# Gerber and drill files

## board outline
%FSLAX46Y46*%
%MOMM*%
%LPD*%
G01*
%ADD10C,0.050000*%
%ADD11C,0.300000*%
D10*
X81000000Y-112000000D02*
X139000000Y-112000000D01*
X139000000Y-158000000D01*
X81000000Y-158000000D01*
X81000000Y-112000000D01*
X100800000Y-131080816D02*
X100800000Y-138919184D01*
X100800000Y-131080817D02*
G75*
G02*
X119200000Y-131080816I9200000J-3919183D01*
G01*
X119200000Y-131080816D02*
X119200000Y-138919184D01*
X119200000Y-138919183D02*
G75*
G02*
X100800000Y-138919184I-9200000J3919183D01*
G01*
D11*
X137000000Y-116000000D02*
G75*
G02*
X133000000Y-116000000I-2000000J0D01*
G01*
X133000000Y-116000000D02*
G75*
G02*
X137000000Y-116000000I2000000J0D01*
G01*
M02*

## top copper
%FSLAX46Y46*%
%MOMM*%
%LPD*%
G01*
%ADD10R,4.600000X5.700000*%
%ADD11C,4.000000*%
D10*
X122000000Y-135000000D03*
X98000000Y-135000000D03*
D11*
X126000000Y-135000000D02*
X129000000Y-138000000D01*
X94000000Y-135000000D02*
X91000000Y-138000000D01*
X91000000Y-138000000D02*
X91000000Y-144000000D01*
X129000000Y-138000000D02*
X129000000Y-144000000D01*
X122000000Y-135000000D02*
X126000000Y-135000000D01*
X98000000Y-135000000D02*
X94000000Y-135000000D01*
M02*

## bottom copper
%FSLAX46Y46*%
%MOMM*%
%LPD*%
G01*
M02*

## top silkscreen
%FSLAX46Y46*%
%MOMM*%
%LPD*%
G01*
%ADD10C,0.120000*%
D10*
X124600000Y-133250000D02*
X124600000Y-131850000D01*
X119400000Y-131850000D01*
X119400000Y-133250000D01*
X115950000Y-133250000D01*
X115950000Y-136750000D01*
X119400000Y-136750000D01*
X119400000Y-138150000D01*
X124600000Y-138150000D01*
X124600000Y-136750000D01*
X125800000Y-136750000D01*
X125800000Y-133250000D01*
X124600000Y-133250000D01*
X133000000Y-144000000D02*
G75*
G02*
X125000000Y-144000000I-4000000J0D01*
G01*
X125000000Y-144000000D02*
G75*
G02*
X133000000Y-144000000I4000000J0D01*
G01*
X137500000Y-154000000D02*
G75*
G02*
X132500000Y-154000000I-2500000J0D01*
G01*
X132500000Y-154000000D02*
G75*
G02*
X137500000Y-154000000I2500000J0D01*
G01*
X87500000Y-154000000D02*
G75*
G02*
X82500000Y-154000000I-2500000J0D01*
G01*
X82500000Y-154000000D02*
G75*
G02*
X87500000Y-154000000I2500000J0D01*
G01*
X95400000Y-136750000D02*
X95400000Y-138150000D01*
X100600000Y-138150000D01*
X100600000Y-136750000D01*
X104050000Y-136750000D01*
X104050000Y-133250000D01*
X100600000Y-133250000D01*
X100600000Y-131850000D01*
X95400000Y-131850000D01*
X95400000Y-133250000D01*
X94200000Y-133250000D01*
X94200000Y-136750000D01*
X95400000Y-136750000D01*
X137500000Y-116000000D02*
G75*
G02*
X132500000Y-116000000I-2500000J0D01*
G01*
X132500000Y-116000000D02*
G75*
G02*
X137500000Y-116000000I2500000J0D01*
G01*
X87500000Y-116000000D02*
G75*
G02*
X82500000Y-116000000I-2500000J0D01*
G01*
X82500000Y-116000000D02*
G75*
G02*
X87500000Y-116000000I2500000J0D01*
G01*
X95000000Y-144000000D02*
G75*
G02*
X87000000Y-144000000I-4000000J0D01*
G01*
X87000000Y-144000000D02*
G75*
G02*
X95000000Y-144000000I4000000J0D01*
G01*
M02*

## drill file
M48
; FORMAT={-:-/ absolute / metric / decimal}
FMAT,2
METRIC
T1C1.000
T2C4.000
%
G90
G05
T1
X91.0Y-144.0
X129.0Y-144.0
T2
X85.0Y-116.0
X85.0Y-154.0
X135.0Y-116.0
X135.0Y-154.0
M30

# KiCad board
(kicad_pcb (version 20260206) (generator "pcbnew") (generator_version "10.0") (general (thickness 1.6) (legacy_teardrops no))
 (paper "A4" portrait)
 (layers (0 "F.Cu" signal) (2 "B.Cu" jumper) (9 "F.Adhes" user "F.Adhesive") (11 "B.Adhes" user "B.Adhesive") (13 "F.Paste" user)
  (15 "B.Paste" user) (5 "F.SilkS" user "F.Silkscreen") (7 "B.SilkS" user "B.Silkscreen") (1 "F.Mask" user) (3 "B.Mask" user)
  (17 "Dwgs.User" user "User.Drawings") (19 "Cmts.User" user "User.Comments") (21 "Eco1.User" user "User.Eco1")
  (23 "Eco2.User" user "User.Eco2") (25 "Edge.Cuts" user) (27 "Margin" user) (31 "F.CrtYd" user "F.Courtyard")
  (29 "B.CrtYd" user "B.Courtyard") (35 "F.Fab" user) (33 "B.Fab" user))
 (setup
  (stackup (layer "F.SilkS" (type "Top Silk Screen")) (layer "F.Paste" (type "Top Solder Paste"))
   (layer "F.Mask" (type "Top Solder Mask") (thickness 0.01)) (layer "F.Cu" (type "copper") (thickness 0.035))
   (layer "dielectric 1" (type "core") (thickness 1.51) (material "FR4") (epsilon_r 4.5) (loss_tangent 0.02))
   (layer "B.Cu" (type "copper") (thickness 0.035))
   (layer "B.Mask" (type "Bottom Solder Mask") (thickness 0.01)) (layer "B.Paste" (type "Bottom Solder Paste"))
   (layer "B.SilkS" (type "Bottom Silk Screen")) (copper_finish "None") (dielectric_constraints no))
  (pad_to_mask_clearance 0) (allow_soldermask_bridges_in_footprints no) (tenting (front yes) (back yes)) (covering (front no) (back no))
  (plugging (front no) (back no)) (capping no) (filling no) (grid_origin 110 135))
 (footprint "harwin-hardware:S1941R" (layer "F.Cu") (at 122 135)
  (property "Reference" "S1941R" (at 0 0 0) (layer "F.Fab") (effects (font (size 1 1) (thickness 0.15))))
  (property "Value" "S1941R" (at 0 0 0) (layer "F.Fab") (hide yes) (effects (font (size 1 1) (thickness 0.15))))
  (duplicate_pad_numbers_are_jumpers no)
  (fp_poly
   (pts (xy 2.6 -1.75) (xy 2.6 -3.15) (xy -2.6 -3.15) (xy -2.6 -1.75) (xy -6.05 -1.75) (xy -6.05 1.75) (xy -2.6 1.75) (xy -2.6 3.15)
    (xy 2.6 3.15) (xy 2.6 1.75) (xy 3.8 1.75) (xy 3.8 -1.75))
   (stroke (width 0.12) (type solid)) (fill no) (layer "F.SilkS"))
  (pad "1" smd rect (at 0 0) (size 4.6 5.7) (layers "F.Cu" "F.Mask" "F.Paste")))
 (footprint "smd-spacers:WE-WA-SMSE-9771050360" (layer "F.Cu") (at 129 144)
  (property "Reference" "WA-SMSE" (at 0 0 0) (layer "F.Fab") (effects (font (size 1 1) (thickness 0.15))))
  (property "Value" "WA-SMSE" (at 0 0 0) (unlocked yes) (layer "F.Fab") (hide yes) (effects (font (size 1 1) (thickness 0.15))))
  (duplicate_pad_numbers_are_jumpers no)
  (fp_circle (center 0 0) (end 4 0) (stroke (width 0.12) (type default)) (fill no) (layer "F.SilkS"))
  (pad "" np_thru_hole circle (at 0 0) (size 1 1) (drill 1) (layers "*.Cu" "*.Mask")))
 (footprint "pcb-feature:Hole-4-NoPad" (layer "F.Cu") (at 135 154)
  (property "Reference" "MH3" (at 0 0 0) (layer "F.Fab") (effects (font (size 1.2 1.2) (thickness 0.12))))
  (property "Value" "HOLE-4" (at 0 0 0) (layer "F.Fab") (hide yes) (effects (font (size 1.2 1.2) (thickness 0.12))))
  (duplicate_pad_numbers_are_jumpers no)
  (fp_circle (center 0 0) (end 2.5 0) (stroke (width 0.12) (type solid)) (fill no) (layer "F.SilkS"))
  (pad "" np_thru_hole circle (at 0 0) (size 4 4) (drill 4) (layers "*.Cu" "*.Mask")))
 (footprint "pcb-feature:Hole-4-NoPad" (layer "F.Cu") (at 85 154)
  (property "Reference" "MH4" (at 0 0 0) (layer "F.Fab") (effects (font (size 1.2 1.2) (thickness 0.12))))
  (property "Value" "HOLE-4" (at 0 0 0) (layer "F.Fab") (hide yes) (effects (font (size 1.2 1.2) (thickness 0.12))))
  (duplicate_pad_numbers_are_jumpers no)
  (fp_circle (center 0 0) (end 2.5 0) (stroke (width 0.12) (type solid)) (fill no) (layer "F.SilkS"))
  (pad "" np_thru_hole circle (at 0 0) (size 4 4) (drill 4) (layers "*.Cu" "*.Mask")))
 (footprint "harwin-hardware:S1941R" (layer "F.Cu") (at 98 135 180)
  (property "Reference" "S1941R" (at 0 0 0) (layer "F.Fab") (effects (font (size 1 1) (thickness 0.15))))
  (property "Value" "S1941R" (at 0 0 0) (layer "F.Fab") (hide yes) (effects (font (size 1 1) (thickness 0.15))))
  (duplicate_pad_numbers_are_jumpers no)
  (fp_poly
   (pts (xy 2.6 -1.75) (xy 2.6 -3.15) (xy -2.6 -3.15) (xy -2.6 -1.75) (xy -6.05 -1.75) (xy -6.05 1.75) (xy -2.6 1.75) (xy -2.6 3.15)
    (xy 2.6 3.15) (xy 2.6 1.75) (xy 3.8 1.75) (xy 3.8 -1.75))
   (stroke (width 0.12) (type solid)) (fill no) (layer "F.SilkS"))
  (pad "1" smd rect (at 0 0 180) (size 4.6 5.7) (layers "F.Cu" "F.Mask" "F.Paste")))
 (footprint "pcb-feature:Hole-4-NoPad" (layer "F.Cu") (at 135 116)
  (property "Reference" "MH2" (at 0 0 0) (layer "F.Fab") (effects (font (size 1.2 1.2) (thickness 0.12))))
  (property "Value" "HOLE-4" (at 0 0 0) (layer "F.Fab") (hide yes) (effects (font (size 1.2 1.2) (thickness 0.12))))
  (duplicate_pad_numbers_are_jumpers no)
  (fp_circle (center 0 0) (end 2.5 0) (stroke (width 0.12) (type solid)) (fill no) (layer "F.SilkS"))
  (pad "" np_thru_hole circle (at 0 0) (size 4 4) (drill 4) (layers "*.Cu" "*.Mask")))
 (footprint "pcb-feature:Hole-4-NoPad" (layer "F.Cu") (at 85 116)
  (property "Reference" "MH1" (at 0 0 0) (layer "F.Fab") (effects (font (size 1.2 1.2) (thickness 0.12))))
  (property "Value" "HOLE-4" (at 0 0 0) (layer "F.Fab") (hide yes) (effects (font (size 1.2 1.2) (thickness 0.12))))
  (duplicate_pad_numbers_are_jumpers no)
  (fp_circle (center 0 0) (end 2.5 0) (stroke (width 0.12) (type solid)) (fill no) (layer "F.SilkS"))
  (pad "" np_thru_hole circle (at 0 0) (size 4 4) (drill 4) (layers "*.Cu" "*.Mask")))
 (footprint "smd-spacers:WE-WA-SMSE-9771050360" (layer "F.Cu") (at 91 144)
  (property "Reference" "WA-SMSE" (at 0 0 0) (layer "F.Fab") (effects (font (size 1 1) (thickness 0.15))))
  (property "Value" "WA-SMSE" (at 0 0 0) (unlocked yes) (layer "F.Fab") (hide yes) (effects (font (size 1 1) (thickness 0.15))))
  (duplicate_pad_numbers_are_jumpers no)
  (fp_circle (center 0 0) (end 4 0) (stroke (width 0.12) (type default)) (fill no) (layer "F.SilkS"))
  (pad "" np_thru_hole circle (at 0 0) (size 1 1) (drill 1) (layers "*.Cu" "*.Mask")))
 (gr_rect (start 81 112) (end 139 158) (stroke (width 0.05) (type default)) (fill no) (layer "Edge.Cuts"))
 (gr_line (start 100.8 131.080816) (end 100.8 138.919184) (stroke (width 0.05) (type solid)) (layer "Edge.Cuts"))
 (gr_arc (start 100.8 131.080817) (mid 110 125) (end 119.2 131.080816) (stroke (width 0.05) (type solid)) (layer "Edge.Cuts"))
 (gr_line (start 119.2 131.080816) (end 119.2 138.919184) (stroke (width 0.05) (type solid)) (layer "Edge.Cuts"))
 (gr_arc (start 119.2 138.919183) (mid 110 145) (end 100.8 138.919184) (stroke (width 0.05) (type solid)) (layer "Edge.Cuts"))
 (gr_circle (center 135 116) (end 133 116) (stroke (width 0.3) (type solid)) (fill no) (layer "Edge.Cuts"))
 (segment (start 126 135) (end 129 138) (width 4) (layer "F.Cu") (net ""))
 (segment (start 94 135) (end 91 138) (width 4) (layer "F.Cu") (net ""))
 (segment (start 91 138) (end 91 144) (width 4) (layer "F.Cu") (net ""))
 (segment (start 129 138) (end 129 144) (width 4) (layer "F.Cu") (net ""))
 (segment (start 122 135) (end 126 135) (width 4) (layer "F.Cu") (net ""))
 (segment (start 98 135) (end 94 135) (width 4) (layer "F.Cu") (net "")))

